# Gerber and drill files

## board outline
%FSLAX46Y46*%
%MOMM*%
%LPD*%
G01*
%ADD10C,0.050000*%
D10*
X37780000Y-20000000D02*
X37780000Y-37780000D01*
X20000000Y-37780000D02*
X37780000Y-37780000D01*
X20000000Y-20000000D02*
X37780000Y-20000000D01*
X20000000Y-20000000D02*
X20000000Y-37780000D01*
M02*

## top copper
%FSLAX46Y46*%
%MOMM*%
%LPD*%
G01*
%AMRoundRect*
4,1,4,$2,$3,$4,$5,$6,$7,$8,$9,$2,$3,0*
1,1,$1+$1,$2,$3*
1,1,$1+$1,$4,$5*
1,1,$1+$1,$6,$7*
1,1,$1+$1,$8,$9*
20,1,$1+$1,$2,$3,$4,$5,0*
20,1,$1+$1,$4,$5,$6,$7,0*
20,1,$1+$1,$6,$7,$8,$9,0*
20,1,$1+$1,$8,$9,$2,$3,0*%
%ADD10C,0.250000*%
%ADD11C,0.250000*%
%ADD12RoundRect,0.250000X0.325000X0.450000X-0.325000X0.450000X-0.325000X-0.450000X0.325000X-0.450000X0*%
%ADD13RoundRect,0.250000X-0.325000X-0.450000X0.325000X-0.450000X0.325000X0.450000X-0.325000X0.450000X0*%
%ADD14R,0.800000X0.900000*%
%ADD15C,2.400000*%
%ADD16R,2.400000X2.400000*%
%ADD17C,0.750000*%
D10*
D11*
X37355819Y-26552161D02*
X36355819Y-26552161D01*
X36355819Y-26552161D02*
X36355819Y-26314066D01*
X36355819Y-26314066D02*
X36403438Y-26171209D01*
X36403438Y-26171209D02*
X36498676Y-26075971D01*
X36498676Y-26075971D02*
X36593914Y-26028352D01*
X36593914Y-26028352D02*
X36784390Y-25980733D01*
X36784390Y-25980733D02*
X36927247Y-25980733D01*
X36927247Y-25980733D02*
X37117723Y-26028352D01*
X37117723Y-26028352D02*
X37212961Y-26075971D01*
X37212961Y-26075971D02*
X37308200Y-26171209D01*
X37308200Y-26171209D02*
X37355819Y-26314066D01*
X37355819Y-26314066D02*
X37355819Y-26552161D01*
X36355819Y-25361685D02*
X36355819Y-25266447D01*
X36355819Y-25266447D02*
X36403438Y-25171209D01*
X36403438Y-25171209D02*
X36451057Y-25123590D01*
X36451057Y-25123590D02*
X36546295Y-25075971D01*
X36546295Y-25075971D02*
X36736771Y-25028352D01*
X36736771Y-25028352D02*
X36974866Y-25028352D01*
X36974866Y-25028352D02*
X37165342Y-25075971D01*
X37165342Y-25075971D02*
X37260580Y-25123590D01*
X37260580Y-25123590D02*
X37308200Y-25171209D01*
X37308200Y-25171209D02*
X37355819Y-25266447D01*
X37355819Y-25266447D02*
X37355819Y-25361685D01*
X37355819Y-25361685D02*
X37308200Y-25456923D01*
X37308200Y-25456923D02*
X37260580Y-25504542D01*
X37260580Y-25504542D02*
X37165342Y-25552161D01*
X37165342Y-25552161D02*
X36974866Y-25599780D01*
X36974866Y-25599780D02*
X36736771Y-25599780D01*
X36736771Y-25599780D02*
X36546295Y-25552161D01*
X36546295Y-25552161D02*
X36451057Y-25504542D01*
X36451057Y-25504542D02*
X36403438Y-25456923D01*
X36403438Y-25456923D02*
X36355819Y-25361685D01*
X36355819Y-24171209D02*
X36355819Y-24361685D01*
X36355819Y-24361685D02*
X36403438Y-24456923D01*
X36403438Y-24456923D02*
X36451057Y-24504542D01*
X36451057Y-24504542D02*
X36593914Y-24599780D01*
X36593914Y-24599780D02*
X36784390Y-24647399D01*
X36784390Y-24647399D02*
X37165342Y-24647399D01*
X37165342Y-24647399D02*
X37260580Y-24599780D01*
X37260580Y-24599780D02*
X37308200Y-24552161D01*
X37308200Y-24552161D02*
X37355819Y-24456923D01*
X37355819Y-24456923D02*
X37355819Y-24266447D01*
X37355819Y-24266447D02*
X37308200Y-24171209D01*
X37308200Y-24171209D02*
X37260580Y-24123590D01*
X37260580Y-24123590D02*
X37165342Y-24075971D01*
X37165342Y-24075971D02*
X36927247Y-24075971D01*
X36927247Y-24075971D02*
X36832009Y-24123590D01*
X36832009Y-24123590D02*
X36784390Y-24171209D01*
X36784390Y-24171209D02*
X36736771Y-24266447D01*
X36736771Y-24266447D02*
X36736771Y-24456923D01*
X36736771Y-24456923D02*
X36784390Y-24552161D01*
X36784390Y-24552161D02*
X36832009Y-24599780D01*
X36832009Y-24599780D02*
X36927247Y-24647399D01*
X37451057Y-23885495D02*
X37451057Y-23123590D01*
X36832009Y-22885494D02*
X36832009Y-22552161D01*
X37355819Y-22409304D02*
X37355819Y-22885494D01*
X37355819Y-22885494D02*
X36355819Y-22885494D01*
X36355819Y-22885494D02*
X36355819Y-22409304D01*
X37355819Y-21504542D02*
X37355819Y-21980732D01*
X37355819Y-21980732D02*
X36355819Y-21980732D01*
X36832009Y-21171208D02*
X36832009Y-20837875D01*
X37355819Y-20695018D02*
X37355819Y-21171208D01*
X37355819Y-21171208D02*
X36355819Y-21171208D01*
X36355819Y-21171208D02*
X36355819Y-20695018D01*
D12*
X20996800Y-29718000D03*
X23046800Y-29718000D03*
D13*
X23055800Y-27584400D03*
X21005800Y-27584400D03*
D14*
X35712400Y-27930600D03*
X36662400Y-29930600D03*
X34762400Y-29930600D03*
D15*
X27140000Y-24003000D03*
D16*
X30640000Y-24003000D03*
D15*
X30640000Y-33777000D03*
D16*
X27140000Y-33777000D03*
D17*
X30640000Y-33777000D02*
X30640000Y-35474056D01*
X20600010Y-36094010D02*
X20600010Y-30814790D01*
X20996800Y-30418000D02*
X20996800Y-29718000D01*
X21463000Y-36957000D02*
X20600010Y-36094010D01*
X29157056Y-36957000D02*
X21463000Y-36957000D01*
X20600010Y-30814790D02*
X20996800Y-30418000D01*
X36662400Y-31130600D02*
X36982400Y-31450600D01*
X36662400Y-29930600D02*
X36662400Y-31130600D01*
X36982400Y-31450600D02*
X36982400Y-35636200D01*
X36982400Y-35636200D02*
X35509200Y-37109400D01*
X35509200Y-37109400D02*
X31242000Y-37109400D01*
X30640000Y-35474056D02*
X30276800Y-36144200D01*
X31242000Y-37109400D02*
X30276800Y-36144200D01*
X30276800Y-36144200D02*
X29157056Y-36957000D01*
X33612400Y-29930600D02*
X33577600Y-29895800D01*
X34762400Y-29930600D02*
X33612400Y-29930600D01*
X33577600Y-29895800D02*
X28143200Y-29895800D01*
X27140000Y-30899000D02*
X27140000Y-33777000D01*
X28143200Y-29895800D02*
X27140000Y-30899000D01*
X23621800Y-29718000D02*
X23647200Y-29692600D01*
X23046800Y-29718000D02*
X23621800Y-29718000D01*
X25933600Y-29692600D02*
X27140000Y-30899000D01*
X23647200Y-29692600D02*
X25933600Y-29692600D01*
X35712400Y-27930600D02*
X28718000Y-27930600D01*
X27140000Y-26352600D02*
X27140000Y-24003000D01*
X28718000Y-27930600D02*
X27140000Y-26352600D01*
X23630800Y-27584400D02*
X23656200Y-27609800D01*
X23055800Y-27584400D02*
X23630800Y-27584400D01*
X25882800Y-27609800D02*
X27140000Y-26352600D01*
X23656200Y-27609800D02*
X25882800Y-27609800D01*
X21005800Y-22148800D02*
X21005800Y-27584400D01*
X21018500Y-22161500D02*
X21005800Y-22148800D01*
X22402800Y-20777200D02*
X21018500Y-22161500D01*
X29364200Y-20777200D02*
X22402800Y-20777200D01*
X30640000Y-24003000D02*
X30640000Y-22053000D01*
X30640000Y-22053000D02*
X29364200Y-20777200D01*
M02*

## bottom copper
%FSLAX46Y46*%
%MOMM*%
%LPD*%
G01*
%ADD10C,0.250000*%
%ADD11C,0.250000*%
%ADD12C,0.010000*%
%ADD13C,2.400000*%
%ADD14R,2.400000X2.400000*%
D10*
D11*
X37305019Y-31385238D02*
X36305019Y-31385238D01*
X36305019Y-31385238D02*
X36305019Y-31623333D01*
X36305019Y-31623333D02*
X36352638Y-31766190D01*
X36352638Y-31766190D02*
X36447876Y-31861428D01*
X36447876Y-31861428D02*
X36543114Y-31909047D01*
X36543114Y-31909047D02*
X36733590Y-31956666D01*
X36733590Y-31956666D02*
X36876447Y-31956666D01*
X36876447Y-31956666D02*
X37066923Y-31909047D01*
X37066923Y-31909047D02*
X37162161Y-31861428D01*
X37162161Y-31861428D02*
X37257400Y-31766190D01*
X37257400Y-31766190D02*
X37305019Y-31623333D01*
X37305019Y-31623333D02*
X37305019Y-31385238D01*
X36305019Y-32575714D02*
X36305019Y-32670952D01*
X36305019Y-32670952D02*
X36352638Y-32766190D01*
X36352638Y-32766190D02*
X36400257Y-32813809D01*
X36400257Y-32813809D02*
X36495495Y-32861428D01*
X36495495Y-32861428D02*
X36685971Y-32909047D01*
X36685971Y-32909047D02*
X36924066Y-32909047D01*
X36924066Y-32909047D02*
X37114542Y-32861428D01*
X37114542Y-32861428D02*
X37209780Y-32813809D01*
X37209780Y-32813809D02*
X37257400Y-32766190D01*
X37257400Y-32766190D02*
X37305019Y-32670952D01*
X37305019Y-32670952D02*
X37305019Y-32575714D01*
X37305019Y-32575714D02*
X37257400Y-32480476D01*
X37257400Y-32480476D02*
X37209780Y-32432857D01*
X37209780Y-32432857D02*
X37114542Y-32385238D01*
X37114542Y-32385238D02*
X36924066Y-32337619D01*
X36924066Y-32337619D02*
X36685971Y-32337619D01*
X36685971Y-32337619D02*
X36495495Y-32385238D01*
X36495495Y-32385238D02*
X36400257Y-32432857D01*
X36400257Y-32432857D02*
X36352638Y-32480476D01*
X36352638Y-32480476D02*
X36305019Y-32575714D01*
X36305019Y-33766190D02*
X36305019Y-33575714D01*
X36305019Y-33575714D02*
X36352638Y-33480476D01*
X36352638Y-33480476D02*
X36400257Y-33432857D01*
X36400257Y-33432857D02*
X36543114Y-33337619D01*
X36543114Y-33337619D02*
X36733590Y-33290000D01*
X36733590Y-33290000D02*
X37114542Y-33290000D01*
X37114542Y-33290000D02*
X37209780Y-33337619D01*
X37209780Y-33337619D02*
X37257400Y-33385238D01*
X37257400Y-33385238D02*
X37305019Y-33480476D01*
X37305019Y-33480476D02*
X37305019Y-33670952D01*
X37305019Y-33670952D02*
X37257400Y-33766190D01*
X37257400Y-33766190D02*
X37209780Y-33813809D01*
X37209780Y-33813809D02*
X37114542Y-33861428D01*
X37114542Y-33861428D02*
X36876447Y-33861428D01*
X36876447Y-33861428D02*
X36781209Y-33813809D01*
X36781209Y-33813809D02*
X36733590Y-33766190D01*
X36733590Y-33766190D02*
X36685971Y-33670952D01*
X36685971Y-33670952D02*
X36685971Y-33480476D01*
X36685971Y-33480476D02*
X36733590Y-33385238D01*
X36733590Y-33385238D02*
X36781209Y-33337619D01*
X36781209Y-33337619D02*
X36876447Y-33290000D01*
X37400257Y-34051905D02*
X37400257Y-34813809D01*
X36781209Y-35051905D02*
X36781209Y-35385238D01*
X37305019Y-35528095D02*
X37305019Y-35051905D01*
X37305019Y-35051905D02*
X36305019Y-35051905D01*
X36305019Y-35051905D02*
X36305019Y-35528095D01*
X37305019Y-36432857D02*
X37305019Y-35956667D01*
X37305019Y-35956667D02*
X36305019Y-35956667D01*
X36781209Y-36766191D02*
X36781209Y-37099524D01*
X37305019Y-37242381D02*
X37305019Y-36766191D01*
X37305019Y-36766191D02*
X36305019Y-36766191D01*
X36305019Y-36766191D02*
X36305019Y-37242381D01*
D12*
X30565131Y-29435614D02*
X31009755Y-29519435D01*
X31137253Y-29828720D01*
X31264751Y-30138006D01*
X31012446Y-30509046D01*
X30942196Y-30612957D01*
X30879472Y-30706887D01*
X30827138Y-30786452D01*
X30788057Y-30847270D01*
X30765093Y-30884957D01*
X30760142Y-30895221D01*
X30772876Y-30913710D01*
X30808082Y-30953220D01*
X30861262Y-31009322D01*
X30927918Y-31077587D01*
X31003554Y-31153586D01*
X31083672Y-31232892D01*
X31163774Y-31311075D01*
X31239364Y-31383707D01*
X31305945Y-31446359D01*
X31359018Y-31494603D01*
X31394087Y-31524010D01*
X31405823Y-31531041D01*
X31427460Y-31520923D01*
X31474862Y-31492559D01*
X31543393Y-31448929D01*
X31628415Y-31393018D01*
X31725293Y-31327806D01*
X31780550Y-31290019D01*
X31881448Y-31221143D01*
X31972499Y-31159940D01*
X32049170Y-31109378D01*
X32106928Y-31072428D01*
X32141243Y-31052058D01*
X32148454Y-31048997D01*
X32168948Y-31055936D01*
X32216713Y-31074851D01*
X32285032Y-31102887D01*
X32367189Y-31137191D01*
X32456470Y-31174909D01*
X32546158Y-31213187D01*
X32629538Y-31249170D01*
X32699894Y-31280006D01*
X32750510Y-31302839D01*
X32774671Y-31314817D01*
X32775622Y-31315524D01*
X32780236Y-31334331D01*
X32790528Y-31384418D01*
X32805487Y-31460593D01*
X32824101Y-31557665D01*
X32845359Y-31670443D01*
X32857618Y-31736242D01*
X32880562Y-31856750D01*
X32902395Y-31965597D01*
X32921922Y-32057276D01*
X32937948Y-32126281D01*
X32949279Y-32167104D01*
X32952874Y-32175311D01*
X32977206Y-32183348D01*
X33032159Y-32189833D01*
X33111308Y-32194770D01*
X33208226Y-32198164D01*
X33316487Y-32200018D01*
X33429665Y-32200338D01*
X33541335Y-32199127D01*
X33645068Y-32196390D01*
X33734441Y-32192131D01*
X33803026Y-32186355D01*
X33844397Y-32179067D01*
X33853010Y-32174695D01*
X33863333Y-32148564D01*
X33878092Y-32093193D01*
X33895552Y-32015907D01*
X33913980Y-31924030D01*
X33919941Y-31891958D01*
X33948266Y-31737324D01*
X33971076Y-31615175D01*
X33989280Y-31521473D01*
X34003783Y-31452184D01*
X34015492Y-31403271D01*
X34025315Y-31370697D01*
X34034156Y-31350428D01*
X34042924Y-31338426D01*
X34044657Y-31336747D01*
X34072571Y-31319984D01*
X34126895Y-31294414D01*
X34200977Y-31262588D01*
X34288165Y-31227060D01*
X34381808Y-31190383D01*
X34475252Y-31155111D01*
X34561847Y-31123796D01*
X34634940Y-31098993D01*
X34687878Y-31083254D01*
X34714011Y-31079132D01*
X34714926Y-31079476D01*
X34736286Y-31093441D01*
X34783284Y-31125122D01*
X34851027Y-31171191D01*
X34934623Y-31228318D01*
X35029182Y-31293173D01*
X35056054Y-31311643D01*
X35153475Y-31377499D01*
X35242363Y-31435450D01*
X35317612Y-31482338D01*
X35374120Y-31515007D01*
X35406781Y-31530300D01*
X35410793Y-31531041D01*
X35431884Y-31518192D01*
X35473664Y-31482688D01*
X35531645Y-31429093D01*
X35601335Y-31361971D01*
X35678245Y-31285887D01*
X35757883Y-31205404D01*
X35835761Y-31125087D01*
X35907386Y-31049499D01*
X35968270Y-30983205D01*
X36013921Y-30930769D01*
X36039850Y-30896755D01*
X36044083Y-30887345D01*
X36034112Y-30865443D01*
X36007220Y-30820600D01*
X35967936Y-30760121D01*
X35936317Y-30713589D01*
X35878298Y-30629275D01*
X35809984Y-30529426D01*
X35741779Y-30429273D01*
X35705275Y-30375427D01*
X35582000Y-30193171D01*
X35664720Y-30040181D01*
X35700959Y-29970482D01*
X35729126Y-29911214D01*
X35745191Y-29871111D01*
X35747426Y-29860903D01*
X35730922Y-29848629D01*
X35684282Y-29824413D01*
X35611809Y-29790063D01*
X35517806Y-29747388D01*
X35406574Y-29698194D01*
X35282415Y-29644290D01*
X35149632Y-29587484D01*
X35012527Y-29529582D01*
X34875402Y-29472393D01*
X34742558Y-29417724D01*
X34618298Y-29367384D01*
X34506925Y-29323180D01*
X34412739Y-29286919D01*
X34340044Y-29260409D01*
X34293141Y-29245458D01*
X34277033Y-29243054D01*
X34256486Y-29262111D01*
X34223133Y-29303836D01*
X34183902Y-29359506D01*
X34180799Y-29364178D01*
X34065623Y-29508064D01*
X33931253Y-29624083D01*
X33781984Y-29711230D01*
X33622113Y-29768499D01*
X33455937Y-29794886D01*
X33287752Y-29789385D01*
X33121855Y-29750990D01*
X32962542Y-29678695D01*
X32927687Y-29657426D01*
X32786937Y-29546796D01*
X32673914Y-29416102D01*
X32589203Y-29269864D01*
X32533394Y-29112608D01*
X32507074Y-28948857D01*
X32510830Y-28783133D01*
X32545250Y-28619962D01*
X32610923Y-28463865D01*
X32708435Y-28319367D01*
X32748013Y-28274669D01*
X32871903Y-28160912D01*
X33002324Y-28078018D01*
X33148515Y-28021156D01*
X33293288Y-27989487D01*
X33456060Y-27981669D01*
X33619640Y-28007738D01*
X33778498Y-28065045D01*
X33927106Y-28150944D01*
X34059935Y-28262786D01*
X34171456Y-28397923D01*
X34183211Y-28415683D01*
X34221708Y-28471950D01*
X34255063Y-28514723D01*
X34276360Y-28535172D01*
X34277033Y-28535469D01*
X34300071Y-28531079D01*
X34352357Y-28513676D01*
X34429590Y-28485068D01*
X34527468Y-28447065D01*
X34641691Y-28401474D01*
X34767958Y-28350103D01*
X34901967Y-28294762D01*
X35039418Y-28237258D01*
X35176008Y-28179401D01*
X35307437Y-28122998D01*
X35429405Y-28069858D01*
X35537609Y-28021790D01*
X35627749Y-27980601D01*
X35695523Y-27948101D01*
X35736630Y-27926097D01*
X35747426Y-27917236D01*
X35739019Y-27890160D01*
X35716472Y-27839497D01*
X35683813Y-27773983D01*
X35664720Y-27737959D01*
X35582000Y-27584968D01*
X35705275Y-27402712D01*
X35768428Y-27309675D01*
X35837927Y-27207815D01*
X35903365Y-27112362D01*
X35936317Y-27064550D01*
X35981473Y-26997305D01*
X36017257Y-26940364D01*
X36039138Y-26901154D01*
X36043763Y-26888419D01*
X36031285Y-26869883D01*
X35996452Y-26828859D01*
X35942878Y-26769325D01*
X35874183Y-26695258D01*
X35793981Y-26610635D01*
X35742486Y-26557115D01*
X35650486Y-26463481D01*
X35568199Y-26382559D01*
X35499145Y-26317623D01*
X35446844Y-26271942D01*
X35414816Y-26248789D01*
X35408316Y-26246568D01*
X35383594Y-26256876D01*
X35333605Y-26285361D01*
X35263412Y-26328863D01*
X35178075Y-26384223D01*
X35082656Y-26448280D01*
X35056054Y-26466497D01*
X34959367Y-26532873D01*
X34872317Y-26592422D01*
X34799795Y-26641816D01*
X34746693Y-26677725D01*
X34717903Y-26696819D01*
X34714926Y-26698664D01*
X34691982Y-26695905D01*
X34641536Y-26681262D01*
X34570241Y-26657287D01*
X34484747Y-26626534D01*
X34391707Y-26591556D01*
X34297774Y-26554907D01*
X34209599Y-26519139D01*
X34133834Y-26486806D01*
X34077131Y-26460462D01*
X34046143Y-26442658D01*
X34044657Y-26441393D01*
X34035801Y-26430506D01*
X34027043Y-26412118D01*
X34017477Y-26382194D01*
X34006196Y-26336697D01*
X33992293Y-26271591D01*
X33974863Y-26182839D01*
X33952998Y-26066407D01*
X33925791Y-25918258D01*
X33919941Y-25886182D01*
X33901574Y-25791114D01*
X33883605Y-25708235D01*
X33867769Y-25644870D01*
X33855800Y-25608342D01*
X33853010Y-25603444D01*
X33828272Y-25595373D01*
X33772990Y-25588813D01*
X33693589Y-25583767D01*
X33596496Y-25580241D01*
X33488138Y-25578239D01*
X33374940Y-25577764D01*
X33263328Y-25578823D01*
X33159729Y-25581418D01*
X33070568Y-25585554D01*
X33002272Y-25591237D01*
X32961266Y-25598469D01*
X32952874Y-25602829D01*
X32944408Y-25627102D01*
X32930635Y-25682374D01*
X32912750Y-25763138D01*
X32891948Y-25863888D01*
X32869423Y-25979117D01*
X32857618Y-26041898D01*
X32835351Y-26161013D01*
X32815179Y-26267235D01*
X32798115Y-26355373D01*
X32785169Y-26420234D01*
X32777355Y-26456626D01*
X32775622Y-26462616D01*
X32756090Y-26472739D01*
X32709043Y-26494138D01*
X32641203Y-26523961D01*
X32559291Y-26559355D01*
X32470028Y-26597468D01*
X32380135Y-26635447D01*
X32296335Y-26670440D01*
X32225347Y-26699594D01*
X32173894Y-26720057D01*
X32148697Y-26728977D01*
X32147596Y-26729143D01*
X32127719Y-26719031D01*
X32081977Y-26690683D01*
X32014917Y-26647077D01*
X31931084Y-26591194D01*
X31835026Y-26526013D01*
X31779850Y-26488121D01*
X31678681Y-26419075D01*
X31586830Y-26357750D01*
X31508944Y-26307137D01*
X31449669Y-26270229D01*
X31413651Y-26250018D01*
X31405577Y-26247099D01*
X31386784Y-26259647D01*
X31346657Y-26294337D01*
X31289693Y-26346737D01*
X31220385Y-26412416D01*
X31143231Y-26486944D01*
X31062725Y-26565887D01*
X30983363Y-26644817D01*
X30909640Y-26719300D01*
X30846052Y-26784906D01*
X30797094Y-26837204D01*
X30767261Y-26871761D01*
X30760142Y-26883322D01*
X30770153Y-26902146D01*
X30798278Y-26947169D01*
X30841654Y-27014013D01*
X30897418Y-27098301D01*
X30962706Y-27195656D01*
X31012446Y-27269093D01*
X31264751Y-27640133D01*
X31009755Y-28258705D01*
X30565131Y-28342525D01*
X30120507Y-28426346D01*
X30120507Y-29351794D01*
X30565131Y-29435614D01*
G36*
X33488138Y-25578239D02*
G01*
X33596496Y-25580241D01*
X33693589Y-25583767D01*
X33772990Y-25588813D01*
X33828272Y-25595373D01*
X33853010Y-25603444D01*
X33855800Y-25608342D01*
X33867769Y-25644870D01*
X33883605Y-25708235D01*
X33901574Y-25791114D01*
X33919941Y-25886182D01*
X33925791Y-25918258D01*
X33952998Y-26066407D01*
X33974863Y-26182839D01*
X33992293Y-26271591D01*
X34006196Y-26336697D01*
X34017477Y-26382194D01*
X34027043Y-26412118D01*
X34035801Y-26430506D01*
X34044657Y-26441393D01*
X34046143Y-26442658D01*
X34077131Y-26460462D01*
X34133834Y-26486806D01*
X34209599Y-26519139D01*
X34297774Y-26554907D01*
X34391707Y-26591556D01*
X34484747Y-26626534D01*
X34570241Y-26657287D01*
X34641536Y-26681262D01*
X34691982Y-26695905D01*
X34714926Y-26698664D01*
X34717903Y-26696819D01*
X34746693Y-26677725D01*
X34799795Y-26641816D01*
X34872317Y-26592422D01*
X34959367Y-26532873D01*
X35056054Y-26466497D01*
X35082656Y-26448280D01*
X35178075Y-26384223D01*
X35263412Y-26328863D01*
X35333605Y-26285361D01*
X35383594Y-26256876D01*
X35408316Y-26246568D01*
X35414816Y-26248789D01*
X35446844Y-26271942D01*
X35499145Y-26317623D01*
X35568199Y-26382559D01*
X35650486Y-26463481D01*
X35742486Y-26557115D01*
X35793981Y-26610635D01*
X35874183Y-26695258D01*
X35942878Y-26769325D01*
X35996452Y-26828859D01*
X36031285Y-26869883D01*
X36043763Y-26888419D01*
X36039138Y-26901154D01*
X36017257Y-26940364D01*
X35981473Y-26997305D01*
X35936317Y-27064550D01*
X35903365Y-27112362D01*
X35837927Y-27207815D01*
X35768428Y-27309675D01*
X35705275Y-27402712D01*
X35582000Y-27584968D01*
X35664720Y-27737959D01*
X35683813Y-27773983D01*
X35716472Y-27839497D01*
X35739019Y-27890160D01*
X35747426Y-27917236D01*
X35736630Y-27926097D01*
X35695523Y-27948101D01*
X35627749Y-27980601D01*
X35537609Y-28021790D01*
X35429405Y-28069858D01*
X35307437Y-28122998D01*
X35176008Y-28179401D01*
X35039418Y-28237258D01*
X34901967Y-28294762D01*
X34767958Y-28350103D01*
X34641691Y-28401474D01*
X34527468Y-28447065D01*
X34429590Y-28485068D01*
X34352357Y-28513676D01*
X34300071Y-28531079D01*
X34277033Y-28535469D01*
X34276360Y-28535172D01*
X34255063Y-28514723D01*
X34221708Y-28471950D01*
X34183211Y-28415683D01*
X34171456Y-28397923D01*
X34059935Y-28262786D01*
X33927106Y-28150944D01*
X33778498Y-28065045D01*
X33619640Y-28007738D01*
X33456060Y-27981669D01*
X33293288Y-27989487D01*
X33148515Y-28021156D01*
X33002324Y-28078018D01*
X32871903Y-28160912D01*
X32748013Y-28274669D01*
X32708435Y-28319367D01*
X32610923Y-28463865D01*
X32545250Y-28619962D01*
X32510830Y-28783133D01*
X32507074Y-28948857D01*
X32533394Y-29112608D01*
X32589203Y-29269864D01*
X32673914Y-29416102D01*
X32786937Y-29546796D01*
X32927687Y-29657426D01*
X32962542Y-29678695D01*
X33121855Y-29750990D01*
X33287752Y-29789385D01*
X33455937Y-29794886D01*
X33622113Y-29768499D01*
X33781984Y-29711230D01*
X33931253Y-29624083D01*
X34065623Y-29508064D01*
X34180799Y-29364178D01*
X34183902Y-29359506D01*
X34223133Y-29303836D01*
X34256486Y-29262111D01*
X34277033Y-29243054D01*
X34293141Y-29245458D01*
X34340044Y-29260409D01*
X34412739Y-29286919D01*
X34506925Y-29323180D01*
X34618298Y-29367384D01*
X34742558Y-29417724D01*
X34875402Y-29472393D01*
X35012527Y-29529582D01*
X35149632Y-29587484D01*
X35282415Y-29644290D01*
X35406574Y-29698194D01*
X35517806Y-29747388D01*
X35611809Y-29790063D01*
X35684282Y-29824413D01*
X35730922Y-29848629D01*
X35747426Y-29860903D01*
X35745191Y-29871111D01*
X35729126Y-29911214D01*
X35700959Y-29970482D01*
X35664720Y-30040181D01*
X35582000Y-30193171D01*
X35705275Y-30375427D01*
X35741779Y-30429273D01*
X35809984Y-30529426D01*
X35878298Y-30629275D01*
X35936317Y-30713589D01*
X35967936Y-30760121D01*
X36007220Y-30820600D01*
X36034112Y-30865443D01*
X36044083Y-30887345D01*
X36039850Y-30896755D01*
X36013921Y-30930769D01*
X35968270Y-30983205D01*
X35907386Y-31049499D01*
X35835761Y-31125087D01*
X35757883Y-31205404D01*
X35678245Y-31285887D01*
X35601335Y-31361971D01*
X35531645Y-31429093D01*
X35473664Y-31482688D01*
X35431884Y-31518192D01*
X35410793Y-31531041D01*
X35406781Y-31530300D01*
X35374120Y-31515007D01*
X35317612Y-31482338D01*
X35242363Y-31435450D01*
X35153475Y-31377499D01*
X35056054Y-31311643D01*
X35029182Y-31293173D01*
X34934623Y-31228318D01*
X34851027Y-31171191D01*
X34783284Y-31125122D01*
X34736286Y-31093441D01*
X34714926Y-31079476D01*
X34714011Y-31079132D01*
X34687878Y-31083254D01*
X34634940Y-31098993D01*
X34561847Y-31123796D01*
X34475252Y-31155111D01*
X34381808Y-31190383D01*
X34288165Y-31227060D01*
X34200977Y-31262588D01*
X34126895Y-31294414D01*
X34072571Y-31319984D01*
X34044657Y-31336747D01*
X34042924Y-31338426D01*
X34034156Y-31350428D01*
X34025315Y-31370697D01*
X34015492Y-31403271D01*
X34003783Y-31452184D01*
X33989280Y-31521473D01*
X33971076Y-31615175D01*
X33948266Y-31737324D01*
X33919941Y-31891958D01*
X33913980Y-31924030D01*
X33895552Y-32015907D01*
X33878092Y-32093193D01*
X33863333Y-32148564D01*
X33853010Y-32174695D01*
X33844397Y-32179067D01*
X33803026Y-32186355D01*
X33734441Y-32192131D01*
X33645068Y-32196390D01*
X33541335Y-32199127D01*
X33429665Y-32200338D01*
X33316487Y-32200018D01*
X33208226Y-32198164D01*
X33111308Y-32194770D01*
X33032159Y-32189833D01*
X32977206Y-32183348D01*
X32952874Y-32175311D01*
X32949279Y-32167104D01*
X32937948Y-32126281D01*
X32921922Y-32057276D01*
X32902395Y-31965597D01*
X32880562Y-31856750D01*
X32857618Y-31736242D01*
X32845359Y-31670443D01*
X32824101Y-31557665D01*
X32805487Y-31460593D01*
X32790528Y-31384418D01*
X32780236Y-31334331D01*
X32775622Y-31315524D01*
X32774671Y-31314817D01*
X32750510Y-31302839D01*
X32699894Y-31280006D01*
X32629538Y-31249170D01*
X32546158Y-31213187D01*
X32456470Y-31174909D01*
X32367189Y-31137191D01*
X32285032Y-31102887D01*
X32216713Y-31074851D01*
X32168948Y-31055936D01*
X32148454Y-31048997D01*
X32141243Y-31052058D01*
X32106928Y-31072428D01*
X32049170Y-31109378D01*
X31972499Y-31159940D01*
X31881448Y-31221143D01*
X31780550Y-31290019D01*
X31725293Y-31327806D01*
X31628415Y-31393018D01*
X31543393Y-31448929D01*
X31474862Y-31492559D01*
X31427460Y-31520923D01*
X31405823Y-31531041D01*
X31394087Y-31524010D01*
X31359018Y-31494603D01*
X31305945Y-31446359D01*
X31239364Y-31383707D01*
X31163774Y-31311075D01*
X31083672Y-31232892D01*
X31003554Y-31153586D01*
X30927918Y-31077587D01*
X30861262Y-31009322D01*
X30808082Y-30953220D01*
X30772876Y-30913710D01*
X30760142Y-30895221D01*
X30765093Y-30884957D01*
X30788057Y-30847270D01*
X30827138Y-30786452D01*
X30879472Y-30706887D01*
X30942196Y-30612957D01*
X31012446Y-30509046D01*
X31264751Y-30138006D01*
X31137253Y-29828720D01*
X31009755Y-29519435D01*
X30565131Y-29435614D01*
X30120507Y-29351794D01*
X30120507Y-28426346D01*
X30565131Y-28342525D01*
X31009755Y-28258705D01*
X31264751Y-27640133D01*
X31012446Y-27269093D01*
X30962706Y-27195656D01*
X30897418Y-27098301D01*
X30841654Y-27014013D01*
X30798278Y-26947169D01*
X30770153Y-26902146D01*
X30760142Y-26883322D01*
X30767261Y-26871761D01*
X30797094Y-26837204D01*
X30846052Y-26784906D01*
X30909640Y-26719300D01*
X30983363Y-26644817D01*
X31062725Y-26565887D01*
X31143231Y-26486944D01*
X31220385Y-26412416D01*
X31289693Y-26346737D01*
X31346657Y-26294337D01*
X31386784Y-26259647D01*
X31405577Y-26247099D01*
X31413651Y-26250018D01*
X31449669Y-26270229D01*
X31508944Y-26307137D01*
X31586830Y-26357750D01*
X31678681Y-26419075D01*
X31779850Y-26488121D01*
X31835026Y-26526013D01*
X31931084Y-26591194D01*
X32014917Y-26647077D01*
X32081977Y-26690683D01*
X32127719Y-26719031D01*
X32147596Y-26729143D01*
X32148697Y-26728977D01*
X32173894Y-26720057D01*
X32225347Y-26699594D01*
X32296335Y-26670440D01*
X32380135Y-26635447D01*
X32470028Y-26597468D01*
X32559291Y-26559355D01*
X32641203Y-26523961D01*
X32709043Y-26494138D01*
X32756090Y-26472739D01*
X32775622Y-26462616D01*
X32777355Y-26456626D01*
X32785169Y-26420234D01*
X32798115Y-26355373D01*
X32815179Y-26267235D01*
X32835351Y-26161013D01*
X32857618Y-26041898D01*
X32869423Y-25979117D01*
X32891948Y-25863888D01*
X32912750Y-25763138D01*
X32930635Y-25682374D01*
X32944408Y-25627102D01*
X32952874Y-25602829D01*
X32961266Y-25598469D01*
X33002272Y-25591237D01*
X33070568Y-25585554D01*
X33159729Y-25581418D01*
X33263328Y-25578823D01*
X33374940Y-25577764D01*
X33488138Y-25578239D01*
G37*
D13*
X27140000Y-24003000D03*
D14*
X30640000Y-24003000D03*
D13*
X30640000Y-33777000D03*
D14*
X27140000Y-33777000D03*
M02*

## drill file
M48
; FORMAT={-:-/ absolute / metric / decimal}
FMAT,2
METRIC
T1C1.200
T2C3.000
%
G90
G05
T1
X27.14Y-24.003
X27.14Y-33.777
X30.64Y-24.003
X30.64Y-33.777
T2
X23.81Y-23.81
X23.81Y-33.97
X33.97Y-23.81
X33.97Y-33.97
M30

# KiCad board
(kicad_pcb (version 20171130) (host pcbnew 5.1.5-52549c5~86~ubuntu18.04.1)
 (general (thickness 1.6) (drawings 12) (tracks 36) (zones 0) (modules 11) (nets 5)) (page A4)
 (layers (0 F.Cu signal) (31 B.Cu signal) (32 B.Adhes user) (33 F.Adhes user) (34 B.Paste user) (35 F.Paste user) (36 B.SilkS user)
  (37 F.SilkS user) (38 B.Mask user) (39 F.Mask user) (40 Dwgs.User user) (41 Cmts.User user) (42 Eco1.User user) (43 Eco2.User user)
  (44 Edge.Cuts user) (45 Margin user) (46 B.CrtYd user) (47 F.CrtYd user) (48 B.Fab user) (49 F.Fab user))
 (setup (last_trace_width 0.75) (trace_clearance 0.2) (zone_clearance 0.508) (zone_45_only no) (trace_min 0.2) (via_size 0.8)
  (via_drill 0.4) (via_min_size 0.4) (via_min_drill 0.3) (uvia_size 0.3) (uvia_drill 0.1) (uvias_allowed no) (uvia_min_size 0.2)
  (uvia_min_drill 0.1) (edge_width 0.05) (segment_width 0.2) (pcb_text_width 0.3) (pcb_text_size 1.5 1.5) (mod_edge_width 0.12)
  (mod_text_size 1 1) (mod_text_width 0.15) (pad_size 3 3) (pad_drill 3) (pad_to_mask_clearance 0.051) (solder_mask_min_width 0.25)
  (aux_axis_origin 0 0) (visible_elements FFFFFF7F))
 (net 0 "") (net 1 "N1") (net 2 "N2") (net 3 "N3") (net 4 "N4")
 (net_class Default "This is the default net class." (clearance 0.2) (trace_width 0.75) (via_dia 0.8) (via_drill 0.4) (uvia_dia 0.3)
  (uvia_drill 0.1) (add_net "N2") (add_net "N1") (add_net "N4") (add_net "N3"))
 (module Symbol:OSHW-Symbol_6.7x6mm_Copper (layer B.Cu) (at 33.0962 28.8798 270)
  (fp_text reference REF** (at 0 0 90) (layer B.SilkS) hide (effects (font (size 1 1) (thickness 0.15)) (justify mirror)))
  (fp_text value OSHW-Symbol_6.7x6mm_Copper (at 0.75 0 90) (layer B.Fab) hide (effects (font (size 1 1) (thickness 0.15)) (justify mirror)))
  (fp_poly
   (pts (xy 0.555814 2.531069) (xy 0.639635 2.086445) (xy 0.94892 1.958947) (xy 1.258206 1.831449) (xy 1.629246 2.083754)
    (xy 1.733157 2.154004) (xy 1.827087 2.216728) (xy 1.906652 2.269062) (xy 1.96747 2.308143) (xy 2.005157 2.331107) (xy 2.015421 2.336058)
    (xy 2.03391 2.323324) (xy 2.07342 2.288118) (xy 2.129522 2.234938) (xy 2.197787 2.168282) (xy 2.273786 2.092646) (xy 2.353092 2.012528)
    (xy 2.431275 1.932426) (xy 2.503907 1.856836) (xy 2.566559 1.790255) (xy 2.614803 1.737182) (xy 2.64421 1.702113) (xy 2.651241 1.690377)
    (xy 2.641123 1.66874) (xy 2.612759 1.621338) (xy 2.569129 1.552807) (xy 2.513218 1.467785) (xy 2.448006 1.370907) (xy 2.410219 1.31565)
    (xy 2.341343 1.214752) (xy 2.28014 1.123701) (xy 2.229578 1.04703) (xy 2.192628 0.989272) (xy 2.172258 0.954957) (xy 2.169197 0.947746)
    (xy 2.176136 0.927252) (xy 2.195051 0.879487) (xy 2.223087 0.811168) (xy 2.257391 0.729011) (xy 2.295109 0.63973) (xy 2.333387 0.550042)
    (xy 2.36937 0.466662) (xy 2.400206 0.396306) (xy 2.423039 0.34569) (xy 2.435017 0.321529) (xy 2.435724 0.320578) (xy 2.454531 0.315964)
    (xy 2.504618 0.305672) (xy 2.580793 0.290713) (xy 2.677865 0.272099) (xy 2.790643 0.250841) (xy 2.856442 0.238582) (xy 2.97695 0.215638)
    (xy 3.085797 0.193805) (xy 3.177476 0.174278) (xy 3.246481 0.158252) (xy 3.287304 0.146921) (xy 3.295511 0.143326)
    (xy 3.303548 0.118994) (xy 3.310033 0.064041) (xy 3.31497 -0.015108) (xy 3.318364 -0.112026) (xy 3.320218 -0.220287)
    (xy 3.320538 -0.333465) (xy 3.319327 -0.445135) (xy 3.31659 -0.548868) (xy 3.312331 -0.638241) (xy 3.306555 -0.706826)
    (xy 3.299267 -0.748197) (xy 3.294895 -0.75681) (xy 3.268764 -0.767133) (xy 3.213393 -0.781892) (xy 3.136107 -0.799352)
    (xy 3.04423 -0.81778) (xy 3.012158 -0.823741) (xy 2.857524 -0.852066) (xy 2.735375 -0.874876) (xy 2.641673 -0.89308)
    (xy 2.572384 -0.907583) (xy 2.523471 -0.919292) (xy 2.490897 -0.929115) (xy 2.470628 -0.937956) (xy 2.458626 -0.946724)
    (xy 2.456947 -0.948457) (xy 2.440184 -0.976371) (xy 2.414614 -1.030695) (xy 2.382788 -1.104777) (xy 2.34726 -1.191965)
    (xy 2.310583 -1.285608) (xy 2.275311 -1.379052) (xy 2.243996 -1.465647) (xy 2.219193 -1.53874) (xy 2.203454 -1.591678)
    (xy 2.199332 -1.617811) (xy 2.199676 -1.618726) (xy 2.213641 -1.640086) (xy 2.245322 -1.687084) (xy 2.291391 -1.754827)
    (xy 2.348518 -1.838423) (xy 2.413373 -1.932982) (xy 2.431843 -1.959854) (xy 2.497699 -2.057275) (xy 2.55565 -2.146163)
    (xy 2.602538 -2.221412) (xy 2.635207 -2.27792) (xy 2.6505 -2.310581) (xy 2.651241 -2.314593) (xy 2.638392 -2.335684)
    (xy 2.602888 -2.377464) (xy 2.549293 -2.435445) (xy 2.482171 -2.505135) (xy 2.406087 -2.582045) (xy 2.325604 -2.661683)
    (xy 2.245287 -2.739561) (xy 2.169699 -2.811186) (xy 2.103405 -2.87207) (xy 2.050969 -2.917721) (xy 2.016955 -2.94365)
    (xy 2.007545 -2.947883) (xy 1.985643 -2.937912) (xy 1.9408 -2.91102) (xy 1.880321 -2.871736) (xy 1.833789 -2.840117)
    (xy 1.749475 -2.782098) (xy 1.649626 -2.713784) (xy 1.549473 -2.645579) (xy 1.495627 -2.609075) (xy 1.313371 -2.4858)
    (xy 1.160381 -2.56852) (xy 1.090682 -2.604759) (xy 1.031414 -2.632926) (xy 0.991311 -2.648991) (xy 0.981103 -2.651226)
    (xy 0.968829 -2.634722) (xy 0.944613 -2.588082) (xy 0.910263 -2.515609) (xy 0.867588 -2.421606) (xy 0.818394 -2.310374)
    (xy 0.76449 -2.186215) (xy 0.707684 -2.053432) (xy 0.649782 -1.916327) (xy 0.592593 -1.779202) (xy 0.537924 -1.646358)
    (xy 0.487584 -1.522098) (xy 0.44338 -1.410725) (xy 0.407119 -1.316539) (xy 0.380609 -1.243844) (xy 0.365658 -1.196941)
    (xy 0.363254 -1.180833) (xy 0.382311 -1.160286) (xy 0.424036 -1.126933) (xy 0.479706 -1.087702) (xy 0.484378 -1.084599)
    (xy 0.628264 -0.969423) (xy 0.744283 -0.835053) (xy 0.83143 -0.685784) (xy 0.888699 -0.525913) (xy 0.915086 -0.359737)
    (xy 0.909585 -0.191552) (xy 0.87119 -0.025655) (xy 0.798895 0.133658) (xy 0.777626 0.168513) (xy 0.666996 0.309263)
    (xy 0.536302 0.422286) (xy 0.390064 0.506997) (xy 0.232808 0.562806) (xy 0.069057 0.589126) (xy -0.096667 0.58537)
    (xy -0.259838 0.55095) (xy -0.415935 0.485277) (xy -0.560433 0.387765) (xy -0.605131 0.348187) (xy -0.718888 0.224297)
    (xy -0.801782 0.093876) (xy -0.858644 -0.052315) (xy -0.890313 -0.197088) (xy -0.898131 -0.35986) (xy -0.872062 -0.52344)
    (xy -0.814755 -0.682298) (xy -0.728856 -0.830906) (xy -0.617014 -0.963735) (xy -0.481877 -1.075256) (xy -0.464117 -1.087011)
    (xy -0.40785 -1.125508) (xy -0.365077 -1.158863) (xy -0.344628 -1.18016) (xy -0.344331 -1.180833) (xy -0.348721 -1.203871)
    (xy -0.366124 -1.256157) (xy -0.394732 -1.33339) (xy -0.432735 -1.431268) (xy -0.478326 -1.545491) (xy -0.529697 -1.671758)
    (xy -0.585038 -1.805767) (xy -0.642542 -1.943218) (xy -0.700399 -2.079808) (xy -0.756802 -2.211237) (xy -0.809942 -2.333205)
    (xy -0.85801 -2.441409) (xy -0.899199 -2.531549) (xy -0.931699 -2.599323) (xy -0.953703 -2.64043) (xy -0.962564 -2.651226)
    (xy -0.98964 -2.642819) (xy -1.040303 -2.620272) (xy -1.105817 -2.587613) (xy -1.141841 -2.56852) (xy -1.294832 -2.4858)
    (xy -1.477088 -2.609075) (xy -1.570125 -2.672228) (xy -1.671985 -2.741727) (xy -1.767438 -2.807165) (xy -1.81525 -2.840117)
    (xy -1.882495 -2.885273) (xy -1.939436 -2.921057) (xy -1.978646 -2.942938) (xy -1.991381 -2.947563) (xy -2.009917 -2.935085)
    (xy -2.050941 -2.900252) (xy -2.110475 -2.846678) (xy -2.184542 -2.777983) (xy -2.269165 -2.697781) (xy -2.322685 -2.646286)
    (xy -2.416319 -2.554286) (xy -2.497241 -2.471999) (xy -2.562177 -2.402945) (xy -2.607858 -2.350644) (xy -2.631011 -2.318616)
    (xy -2.633232 -2.312116) (xy -2.622924 -2.287394) (xy -2.594439 -2.237405) (xy -2.550937 -2.167212) (xy -2.495577 -2.081875)
    (xy -2.43152 -1.986456) (xy -2.413303 -1.959854) (xy -2.346927 -1.863167) (xy -2.287378 -1.776117) (xy -2.237984 -1.703595)
    (xy -2.202075 -1.650493) (xy -2.182981 -1.621703) (xy -2.181136 -1.618726) (xy -2.183895 -1.595782) (xy -2.198538 -1.545336)
    (xy -2.222513 -1.474041) (xy -2.253266 -1.388547) (xy -2.288244 -1.295507) (xy -2.324893 -1.201574) (xy -2.360661 -1.113399)
    (xy -2.392994 -1.037634) (xy -2.419338 -0.980931) (xy -2.437142 -0.949943) (xy -2.438407 -0.948457) (xy -2.449294 -0.939601)
    (xy -2.467682 -0.930843) (xy -2.497606 -0.921277) (xy -2.543103 -0.909996) (xy -2.608209 -0.896093) (xy -2.696961 -0.878663)
    (xy -2.813393 -0.856798) (xy -2.961542 -0.829591) (xy -2.993618 -0.823741) (xy -3.088686 -0.805374) (xy -3.171565 -0.787405)
    (xy -3.23493 -0.771569) (xy -3.271458 -0.7596) (xy -3.276356 -0.75681) (xy -3.284427 -0.732072) (xy -3.290987 -0.67679)
    (xy -3.296033 -0.597389) (xy -3.299559 -0.500296) (xy -3.301561 -0.391938) (xy -3.302036 -0.27874) (xy -3.300977 -0.167128)
    (xy -3.298382 -0.063529) (xy -3.294246 0.025632) (xy -3.288563 0.093928) (xy -3.281331 0.134934) (xy -3.276971 0.143326)
    (xy -3.252698 0.151792) (xy -3.197426 0.165565) (xy -3.116662 0.18345) (xy -3.015912 0.204252) (xy -2.900683 0.226777)
    (xy -2.837902 0.238582) (xy -2.718787 0.260849) (xy -2.612565 0.281021) (xy -2.524427 0.298085) (xy -2.459566 0.311031)
    (xy -2.423174 0.318845) (xy -2.417184 0.320578) (xy -2.407061 0.34011) (xy -2.385662 0.387157) (xy -2.355839 0.454997)
    (xy -2.320445 0.536909) (xy -2.282332 0.626172) (xy -2.244353 0.716065) (xy -2.20936 0.799865) (xy -2.180206 0.870853)
    (xy -2.159743 0.922306) (xy -2.150823 0.947503) (xy -2.150657 0.948604) (xy -2.160769 0.968481) (xy -2.189117 1.014223)
    (xy -2.232723 1.081283) (xy -2.288606 1.165116) (xy -2.353787 1.261174) (xy -2.391679 1.31635) (xy -2.460725 1.417519)
    (xy -2.52205 1.50937) (xy -2.572663 1.587256) (xy -2.609571 1.646531) (xy -2.629782 1.682549) (xy -2.632701 1.690623)
    (xy -2.620153 1.709416) (xy -2.585463 1.749543) (xy -2.533063 1.806507) (xy -2.467384 1.875815) (xy -2.392856 1.952969)
    (xy -2.313913 2.033475) (xy -2.234983 2.112837) (xy -2.1605 2.18656) (xy -2.094894 2.250148) (xy -2.042596 2.299106)
    (xy -2.008039 2.328939) (xy -1.996478 2.336058) (xy -1.977654 2.326047) (xy -1.932631 2.297922) (xy -1.865787 2.254546)
    (xy -1.781499 2.198782) (xy -1.684144 2.133494) (xy -1.610707 2.083754) (xy -1.239667 1.831449) (xy -0.621095 2.086445)
    (xy -0.537275 2.531069) (xy -0.453454 2.975693) (xy 0.471994 2.975693) (xy 0.555814 2.531069))
   (layer B.Cu) (width 0.01)))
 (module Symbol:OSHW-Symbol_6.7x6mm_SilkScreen (layer B.Cu) (at 24.638 28.8544 90)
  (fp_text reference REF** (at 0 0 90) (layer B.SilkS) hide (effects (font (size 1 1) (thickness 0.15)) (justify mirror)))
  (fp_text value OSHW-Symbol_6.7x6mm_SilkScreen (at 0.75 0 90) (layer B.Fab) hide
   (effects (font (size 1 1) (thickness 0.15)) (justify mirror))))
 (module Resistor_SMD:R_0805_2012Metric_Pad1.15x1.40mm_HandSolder (layer F.Cu) (at 22.0218 29.718 180)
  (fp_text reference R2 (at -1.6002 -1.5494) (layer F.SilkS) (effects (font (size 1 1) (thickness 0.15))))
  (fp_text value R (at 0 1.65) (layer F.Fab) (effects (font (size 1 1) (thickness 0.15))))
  (pad 2 smd roundrect (at 1.025 0 180) (size 1.15 1.4) (layers F.Cu F.Paste F.Mask) (roundrect_rratio 0.217391) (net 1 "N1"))
  (pad 1 smd roundrect (at -1.025 0 180) (size 1.15 1.4) (layers F.Cu F.Paste F.Mask) (roundrect_rratio 0.217391) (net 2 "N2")))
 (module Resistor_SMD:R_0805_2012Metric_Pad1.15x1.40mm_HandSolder (layer F.Cu) (at 22.0308 27.5844)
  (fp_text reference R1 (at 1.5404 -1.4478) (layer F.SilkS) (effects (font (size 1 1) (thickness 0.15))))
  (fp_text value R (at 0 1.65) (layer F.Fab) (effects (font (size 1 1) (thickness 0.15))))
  (pad 2 smd roundrect (at 1.025 0) (size 1.15 1.4) (layers F.Cu F.Paste F.Mask) (roundrect_rratio 0.217391) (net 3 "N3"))
  (pad 1 smd roundrect (at -1.025 0) (size 1.15 1.4) (layers F.Cu F.Paste F.Mask) (roundrect_rratio 0.217391) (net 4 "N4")))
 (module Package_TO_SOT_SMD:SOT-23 (layer F.Cu) (at 35.7124 28.9306 90)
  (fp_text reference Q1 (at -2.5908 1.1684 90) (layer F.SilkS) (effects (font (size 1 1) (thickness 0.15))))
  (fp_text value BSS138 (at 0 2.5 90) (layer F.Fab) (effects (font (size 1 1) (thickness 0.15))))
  (pad 3 smd rect (at 1 0 90) (size 0.9 0.8) (layers F.Cu F.Paste F.Mask) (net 3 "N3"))
  (pad 2 smd rect (at -1 0.95 90) (size 0.9 0.8) (layers F.Cu F.Paste F.Mask) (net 1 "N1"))
  (pad 1 smd rect (at -1 -0.95 90) (size 0.9 0.8) (layers F.Cu F.Paste F.Mask) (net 2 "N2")))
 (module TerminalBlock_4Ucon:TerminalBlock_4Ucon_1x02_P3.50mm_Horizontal (layer F.Cu) (at 30.64 24.003 180)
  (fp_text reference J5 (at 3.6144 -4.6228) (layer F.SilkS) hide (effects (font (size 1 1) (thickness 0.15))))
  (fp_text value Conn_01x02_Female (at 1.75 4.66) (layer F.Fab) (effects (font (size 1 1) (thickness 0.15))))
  (pad 2 thru_hole circle (at 3.5 0 180) (size 2.4 2.4) (drill 1.2) (layers *.Cu *.Mask) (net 3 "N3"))
  (pad 1 thru_hole rect (at 0 0 180) (size 2.4 2.4) (drill 1.2) (layers *.Cu *.Mask) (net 4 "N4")))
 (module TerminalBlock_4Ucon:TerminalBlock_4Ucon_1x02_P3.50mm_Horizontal (layer F.Cu) (at 27.14 33.777)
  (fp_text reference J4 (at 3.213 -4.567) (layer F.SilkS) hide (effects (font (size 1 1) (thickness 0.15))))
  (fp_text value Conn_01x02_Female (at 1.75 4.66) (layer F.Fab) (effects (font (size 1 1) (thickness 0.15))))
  (pad 2 thru_hole circle (at 3.5 0) (size 2.4 2.4) (drill 1.2) (layers *.Cu *.Mask) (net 1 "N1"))
  (pad 1 thru_hole rect (at 0 0) (size 2.4 2.4) (drill 1.2) (layers *.Cu *.Mask) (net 2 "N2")))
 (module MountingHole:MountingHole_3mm (layer F.Cu) (at 33.97 33.97)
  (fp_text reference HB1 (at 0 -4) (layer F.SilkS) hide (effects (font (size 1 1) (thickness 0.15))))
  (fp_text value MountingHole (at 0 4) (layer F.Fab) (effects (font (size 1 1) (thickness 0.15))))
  (pad 1 np_thru_hole circle (at 0 0) (size 3 3) (drill 3) (layers *.Cu *.Mask)))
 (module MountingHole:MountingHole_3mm (layer F.Cu) (at 23.81 33.97)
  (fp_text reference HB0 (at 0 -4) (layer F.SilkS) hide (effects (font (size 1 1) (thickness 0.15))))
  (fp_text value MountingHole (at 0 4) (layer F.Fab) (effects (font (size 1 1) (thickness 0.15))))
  (pad 1 np_thru_hole circle (at 0 0) (size 3 3) (drill 3) (layers *.Cu *.Mask)))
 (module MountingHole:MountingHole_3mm (layer F.Cu) (at 33.97 23.81)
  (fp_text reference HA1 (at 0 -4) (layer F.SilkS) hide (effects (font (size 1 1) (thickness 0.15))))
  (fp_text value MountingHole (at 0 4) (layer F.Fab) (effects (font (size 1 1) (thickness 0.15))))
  (pad 1 np_thru_hole circle (at 0 0) (size 3 3) (drill 3) (layers *.Cu *.Mask)))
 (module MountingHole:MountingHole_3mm (layer F.Cu) (at 23.81 23.81)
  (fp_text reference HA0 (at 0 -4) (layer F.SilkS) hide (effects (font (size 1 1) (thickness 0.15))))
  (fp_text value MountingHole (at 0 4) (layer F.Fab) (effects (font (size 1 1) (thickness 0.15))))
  (pad 1 np_thru_hole circle (at 0 0) (size 3 3) (drill 3) (layers *.Cu *.Mask)))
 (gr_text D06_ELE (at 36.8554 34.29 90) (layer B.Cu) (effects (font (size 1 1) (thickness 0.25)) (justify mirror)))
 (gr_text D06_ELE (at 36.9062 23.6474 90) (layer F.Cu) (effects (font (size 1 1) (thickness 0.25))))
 (gr_line (start 37.78 20) (end 37.78 37.78) (layer Edge.Cuts) (width 0.05))
 (gr_line (start 20 37.78) (end 37.78 37.78) (layer Edge.Cuts) (width 0.05))
 (gr_line (start 20 20) (end 37.78 20) (layer Edge.Cuts) (width 0.05))
 (gr_line (start 20 20) (end 20 37.78) (layer Edge.Cuts) (width 0.05))
 (segment (start 30.64 33.777) (end 30.64 35.474056) (width 0.75) (layer F.Cu) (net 1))
 (segment (start 20.60001 36.09401) (end 20.60001 30.81479) (width 0.75) (layer F.Cu) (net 1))
 (segment (start 20.9968 30.418) (end 20.9968 29.718) (width 0.75) (layer F.Cu) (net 1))
 (segment (start 21.463 36.957) (end 20.60001 36.09401) (width 0.75) (layer F.Cu) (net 1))
 (segment (start 29.157056 36.957) (end 21.463 36.957) (width 0.75) (layer F.Cu) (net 1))
 (segment (start 20.60001 30.81479) (end 20.9968 30.418) (width 0.75) (layer F.Cu) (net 1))
 (segment (start 36.6624 31.1306) (end 36.9824 31.4506) (width 0.75) (layer F.Cu) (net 1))
 (segment (start 36.6624 29.9306) (end 36.6624 31.1306) (width 0.75) (layer F.Cu) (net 1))
 (segment (start 36.9824 31.4506) (end 36.9824 35.6362) (width 0.75) (layer F.Cu) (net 1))
 (segment (start 36.9824 35.6362) (end 35.5092 37.1094) (width 0.75) (layer F.Cu) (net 1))
 (segment (start 35.5092 37.1094) (end 31.242 37.1094) (width 0.75) (layer F.Cu) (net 1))
 (segment (start 30.64 35.474056) (end 30.2768 36.1442) (width 0.75) (layer F.Cu) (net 1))
 (segment (start 31.242 37.1094) (end 30.2768 36.1442) (width 0.75) (layer F.Cu) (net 1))
 (segment (start 30.2768 36.1442) (end 29.157056 36.957) (width 0.75) (layer F.Cu) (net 1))
 (segment (start 33.6124 29.9306) (end 33.5776 29.8958) (width 0.75) (layer F.Cu) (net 2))
 (segment (start 34.7624 29.9306) (end 33.6124 29.9306) (width 0.75) (layer F.Cu) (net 2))
 (segment (start 33.5776 29.8958) (end 28.1432 29.8958) (width 0.75) (layer F.Cu) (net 2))
 (segment (start 27.14 30.899) (end 27.14 33.777) (width 0.75) (layer F.Cu) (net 2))
 (segment (start 28.1432 29.8958) (end 27.14 30.899) (width 0.75) (layer F.Cu) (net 2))
 (segment (start 23.6218 29.718) (end 23.6472 29.6926) (width 0.75) (layer F.Cu) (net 2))
 (segment (start 23.0468 29.718) (end 23.6218 29.718) (width 0.75) (layer F.Cu) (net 2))
 (segment (start 25.9336 29.6926) (end 27.14 30.899) (width 0.75) (layer F.Cu) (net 2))
 (segment (start 23.6472 29.6926) (end 25.9336 29.6926) (width 0.75) (layer F.Cu) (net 2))
 (segment (start 35.7124 27.9306) (end 28.718 27.9306) (width 0.75) (layer F.Cu) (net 3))
 (segment (start 27.14 26.3526) (end 27.14 24.003) (width 0.75) (layer F.Cu) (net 3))
 (segment (start 28.718 27.9306) (end 27.14 26.3526) (width 0.75) (layer F.Cu) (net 3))
 (segment (start 23.6308 27.5844) (end 23.6562 27.6098) (width 0.75) (layer F.Cu) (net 3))
 (segment (start 23.0558 27.5844) (end 23.6308 27.5844) (width 0.75) (layer F.Cu) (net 3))
 (segment (start 25.8828 27.6098) (end 27.14 26.3526) (width 0.75) (layer F.Cu) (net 3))
 (segment (start 23.6562 27.6098) (end 25.8828 27.6098) (width 0.75) (layer F.Cu) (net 3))
 (segment (start 21.0058 22.1488) (end 21.0058 27.5844) (width 0.75) (layer F.Cu) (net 4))
 (segment (start 21.0185 22.1615) (end 21.0058 22.1488) (width 0.75) (layer F.Cu) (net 4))
 (segment (start 22.4028 20.7772) (end 21.0185 22.1615) (width 0.75) (layer F.Cu) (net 4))
 (segment (start 29.3642 20.7772) (end 22.4028 20.7772) (width 0.75) (layer F.Cu) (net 4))
 (segment (start 30.64 24.003) (end 30.64 22.053) (width 0.75) (layer F.Cu) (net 4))
 (segment (start 30.64 22.053) (end 29.3642 20.7772) (width 0.75) (layer F.Cu) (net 4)))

